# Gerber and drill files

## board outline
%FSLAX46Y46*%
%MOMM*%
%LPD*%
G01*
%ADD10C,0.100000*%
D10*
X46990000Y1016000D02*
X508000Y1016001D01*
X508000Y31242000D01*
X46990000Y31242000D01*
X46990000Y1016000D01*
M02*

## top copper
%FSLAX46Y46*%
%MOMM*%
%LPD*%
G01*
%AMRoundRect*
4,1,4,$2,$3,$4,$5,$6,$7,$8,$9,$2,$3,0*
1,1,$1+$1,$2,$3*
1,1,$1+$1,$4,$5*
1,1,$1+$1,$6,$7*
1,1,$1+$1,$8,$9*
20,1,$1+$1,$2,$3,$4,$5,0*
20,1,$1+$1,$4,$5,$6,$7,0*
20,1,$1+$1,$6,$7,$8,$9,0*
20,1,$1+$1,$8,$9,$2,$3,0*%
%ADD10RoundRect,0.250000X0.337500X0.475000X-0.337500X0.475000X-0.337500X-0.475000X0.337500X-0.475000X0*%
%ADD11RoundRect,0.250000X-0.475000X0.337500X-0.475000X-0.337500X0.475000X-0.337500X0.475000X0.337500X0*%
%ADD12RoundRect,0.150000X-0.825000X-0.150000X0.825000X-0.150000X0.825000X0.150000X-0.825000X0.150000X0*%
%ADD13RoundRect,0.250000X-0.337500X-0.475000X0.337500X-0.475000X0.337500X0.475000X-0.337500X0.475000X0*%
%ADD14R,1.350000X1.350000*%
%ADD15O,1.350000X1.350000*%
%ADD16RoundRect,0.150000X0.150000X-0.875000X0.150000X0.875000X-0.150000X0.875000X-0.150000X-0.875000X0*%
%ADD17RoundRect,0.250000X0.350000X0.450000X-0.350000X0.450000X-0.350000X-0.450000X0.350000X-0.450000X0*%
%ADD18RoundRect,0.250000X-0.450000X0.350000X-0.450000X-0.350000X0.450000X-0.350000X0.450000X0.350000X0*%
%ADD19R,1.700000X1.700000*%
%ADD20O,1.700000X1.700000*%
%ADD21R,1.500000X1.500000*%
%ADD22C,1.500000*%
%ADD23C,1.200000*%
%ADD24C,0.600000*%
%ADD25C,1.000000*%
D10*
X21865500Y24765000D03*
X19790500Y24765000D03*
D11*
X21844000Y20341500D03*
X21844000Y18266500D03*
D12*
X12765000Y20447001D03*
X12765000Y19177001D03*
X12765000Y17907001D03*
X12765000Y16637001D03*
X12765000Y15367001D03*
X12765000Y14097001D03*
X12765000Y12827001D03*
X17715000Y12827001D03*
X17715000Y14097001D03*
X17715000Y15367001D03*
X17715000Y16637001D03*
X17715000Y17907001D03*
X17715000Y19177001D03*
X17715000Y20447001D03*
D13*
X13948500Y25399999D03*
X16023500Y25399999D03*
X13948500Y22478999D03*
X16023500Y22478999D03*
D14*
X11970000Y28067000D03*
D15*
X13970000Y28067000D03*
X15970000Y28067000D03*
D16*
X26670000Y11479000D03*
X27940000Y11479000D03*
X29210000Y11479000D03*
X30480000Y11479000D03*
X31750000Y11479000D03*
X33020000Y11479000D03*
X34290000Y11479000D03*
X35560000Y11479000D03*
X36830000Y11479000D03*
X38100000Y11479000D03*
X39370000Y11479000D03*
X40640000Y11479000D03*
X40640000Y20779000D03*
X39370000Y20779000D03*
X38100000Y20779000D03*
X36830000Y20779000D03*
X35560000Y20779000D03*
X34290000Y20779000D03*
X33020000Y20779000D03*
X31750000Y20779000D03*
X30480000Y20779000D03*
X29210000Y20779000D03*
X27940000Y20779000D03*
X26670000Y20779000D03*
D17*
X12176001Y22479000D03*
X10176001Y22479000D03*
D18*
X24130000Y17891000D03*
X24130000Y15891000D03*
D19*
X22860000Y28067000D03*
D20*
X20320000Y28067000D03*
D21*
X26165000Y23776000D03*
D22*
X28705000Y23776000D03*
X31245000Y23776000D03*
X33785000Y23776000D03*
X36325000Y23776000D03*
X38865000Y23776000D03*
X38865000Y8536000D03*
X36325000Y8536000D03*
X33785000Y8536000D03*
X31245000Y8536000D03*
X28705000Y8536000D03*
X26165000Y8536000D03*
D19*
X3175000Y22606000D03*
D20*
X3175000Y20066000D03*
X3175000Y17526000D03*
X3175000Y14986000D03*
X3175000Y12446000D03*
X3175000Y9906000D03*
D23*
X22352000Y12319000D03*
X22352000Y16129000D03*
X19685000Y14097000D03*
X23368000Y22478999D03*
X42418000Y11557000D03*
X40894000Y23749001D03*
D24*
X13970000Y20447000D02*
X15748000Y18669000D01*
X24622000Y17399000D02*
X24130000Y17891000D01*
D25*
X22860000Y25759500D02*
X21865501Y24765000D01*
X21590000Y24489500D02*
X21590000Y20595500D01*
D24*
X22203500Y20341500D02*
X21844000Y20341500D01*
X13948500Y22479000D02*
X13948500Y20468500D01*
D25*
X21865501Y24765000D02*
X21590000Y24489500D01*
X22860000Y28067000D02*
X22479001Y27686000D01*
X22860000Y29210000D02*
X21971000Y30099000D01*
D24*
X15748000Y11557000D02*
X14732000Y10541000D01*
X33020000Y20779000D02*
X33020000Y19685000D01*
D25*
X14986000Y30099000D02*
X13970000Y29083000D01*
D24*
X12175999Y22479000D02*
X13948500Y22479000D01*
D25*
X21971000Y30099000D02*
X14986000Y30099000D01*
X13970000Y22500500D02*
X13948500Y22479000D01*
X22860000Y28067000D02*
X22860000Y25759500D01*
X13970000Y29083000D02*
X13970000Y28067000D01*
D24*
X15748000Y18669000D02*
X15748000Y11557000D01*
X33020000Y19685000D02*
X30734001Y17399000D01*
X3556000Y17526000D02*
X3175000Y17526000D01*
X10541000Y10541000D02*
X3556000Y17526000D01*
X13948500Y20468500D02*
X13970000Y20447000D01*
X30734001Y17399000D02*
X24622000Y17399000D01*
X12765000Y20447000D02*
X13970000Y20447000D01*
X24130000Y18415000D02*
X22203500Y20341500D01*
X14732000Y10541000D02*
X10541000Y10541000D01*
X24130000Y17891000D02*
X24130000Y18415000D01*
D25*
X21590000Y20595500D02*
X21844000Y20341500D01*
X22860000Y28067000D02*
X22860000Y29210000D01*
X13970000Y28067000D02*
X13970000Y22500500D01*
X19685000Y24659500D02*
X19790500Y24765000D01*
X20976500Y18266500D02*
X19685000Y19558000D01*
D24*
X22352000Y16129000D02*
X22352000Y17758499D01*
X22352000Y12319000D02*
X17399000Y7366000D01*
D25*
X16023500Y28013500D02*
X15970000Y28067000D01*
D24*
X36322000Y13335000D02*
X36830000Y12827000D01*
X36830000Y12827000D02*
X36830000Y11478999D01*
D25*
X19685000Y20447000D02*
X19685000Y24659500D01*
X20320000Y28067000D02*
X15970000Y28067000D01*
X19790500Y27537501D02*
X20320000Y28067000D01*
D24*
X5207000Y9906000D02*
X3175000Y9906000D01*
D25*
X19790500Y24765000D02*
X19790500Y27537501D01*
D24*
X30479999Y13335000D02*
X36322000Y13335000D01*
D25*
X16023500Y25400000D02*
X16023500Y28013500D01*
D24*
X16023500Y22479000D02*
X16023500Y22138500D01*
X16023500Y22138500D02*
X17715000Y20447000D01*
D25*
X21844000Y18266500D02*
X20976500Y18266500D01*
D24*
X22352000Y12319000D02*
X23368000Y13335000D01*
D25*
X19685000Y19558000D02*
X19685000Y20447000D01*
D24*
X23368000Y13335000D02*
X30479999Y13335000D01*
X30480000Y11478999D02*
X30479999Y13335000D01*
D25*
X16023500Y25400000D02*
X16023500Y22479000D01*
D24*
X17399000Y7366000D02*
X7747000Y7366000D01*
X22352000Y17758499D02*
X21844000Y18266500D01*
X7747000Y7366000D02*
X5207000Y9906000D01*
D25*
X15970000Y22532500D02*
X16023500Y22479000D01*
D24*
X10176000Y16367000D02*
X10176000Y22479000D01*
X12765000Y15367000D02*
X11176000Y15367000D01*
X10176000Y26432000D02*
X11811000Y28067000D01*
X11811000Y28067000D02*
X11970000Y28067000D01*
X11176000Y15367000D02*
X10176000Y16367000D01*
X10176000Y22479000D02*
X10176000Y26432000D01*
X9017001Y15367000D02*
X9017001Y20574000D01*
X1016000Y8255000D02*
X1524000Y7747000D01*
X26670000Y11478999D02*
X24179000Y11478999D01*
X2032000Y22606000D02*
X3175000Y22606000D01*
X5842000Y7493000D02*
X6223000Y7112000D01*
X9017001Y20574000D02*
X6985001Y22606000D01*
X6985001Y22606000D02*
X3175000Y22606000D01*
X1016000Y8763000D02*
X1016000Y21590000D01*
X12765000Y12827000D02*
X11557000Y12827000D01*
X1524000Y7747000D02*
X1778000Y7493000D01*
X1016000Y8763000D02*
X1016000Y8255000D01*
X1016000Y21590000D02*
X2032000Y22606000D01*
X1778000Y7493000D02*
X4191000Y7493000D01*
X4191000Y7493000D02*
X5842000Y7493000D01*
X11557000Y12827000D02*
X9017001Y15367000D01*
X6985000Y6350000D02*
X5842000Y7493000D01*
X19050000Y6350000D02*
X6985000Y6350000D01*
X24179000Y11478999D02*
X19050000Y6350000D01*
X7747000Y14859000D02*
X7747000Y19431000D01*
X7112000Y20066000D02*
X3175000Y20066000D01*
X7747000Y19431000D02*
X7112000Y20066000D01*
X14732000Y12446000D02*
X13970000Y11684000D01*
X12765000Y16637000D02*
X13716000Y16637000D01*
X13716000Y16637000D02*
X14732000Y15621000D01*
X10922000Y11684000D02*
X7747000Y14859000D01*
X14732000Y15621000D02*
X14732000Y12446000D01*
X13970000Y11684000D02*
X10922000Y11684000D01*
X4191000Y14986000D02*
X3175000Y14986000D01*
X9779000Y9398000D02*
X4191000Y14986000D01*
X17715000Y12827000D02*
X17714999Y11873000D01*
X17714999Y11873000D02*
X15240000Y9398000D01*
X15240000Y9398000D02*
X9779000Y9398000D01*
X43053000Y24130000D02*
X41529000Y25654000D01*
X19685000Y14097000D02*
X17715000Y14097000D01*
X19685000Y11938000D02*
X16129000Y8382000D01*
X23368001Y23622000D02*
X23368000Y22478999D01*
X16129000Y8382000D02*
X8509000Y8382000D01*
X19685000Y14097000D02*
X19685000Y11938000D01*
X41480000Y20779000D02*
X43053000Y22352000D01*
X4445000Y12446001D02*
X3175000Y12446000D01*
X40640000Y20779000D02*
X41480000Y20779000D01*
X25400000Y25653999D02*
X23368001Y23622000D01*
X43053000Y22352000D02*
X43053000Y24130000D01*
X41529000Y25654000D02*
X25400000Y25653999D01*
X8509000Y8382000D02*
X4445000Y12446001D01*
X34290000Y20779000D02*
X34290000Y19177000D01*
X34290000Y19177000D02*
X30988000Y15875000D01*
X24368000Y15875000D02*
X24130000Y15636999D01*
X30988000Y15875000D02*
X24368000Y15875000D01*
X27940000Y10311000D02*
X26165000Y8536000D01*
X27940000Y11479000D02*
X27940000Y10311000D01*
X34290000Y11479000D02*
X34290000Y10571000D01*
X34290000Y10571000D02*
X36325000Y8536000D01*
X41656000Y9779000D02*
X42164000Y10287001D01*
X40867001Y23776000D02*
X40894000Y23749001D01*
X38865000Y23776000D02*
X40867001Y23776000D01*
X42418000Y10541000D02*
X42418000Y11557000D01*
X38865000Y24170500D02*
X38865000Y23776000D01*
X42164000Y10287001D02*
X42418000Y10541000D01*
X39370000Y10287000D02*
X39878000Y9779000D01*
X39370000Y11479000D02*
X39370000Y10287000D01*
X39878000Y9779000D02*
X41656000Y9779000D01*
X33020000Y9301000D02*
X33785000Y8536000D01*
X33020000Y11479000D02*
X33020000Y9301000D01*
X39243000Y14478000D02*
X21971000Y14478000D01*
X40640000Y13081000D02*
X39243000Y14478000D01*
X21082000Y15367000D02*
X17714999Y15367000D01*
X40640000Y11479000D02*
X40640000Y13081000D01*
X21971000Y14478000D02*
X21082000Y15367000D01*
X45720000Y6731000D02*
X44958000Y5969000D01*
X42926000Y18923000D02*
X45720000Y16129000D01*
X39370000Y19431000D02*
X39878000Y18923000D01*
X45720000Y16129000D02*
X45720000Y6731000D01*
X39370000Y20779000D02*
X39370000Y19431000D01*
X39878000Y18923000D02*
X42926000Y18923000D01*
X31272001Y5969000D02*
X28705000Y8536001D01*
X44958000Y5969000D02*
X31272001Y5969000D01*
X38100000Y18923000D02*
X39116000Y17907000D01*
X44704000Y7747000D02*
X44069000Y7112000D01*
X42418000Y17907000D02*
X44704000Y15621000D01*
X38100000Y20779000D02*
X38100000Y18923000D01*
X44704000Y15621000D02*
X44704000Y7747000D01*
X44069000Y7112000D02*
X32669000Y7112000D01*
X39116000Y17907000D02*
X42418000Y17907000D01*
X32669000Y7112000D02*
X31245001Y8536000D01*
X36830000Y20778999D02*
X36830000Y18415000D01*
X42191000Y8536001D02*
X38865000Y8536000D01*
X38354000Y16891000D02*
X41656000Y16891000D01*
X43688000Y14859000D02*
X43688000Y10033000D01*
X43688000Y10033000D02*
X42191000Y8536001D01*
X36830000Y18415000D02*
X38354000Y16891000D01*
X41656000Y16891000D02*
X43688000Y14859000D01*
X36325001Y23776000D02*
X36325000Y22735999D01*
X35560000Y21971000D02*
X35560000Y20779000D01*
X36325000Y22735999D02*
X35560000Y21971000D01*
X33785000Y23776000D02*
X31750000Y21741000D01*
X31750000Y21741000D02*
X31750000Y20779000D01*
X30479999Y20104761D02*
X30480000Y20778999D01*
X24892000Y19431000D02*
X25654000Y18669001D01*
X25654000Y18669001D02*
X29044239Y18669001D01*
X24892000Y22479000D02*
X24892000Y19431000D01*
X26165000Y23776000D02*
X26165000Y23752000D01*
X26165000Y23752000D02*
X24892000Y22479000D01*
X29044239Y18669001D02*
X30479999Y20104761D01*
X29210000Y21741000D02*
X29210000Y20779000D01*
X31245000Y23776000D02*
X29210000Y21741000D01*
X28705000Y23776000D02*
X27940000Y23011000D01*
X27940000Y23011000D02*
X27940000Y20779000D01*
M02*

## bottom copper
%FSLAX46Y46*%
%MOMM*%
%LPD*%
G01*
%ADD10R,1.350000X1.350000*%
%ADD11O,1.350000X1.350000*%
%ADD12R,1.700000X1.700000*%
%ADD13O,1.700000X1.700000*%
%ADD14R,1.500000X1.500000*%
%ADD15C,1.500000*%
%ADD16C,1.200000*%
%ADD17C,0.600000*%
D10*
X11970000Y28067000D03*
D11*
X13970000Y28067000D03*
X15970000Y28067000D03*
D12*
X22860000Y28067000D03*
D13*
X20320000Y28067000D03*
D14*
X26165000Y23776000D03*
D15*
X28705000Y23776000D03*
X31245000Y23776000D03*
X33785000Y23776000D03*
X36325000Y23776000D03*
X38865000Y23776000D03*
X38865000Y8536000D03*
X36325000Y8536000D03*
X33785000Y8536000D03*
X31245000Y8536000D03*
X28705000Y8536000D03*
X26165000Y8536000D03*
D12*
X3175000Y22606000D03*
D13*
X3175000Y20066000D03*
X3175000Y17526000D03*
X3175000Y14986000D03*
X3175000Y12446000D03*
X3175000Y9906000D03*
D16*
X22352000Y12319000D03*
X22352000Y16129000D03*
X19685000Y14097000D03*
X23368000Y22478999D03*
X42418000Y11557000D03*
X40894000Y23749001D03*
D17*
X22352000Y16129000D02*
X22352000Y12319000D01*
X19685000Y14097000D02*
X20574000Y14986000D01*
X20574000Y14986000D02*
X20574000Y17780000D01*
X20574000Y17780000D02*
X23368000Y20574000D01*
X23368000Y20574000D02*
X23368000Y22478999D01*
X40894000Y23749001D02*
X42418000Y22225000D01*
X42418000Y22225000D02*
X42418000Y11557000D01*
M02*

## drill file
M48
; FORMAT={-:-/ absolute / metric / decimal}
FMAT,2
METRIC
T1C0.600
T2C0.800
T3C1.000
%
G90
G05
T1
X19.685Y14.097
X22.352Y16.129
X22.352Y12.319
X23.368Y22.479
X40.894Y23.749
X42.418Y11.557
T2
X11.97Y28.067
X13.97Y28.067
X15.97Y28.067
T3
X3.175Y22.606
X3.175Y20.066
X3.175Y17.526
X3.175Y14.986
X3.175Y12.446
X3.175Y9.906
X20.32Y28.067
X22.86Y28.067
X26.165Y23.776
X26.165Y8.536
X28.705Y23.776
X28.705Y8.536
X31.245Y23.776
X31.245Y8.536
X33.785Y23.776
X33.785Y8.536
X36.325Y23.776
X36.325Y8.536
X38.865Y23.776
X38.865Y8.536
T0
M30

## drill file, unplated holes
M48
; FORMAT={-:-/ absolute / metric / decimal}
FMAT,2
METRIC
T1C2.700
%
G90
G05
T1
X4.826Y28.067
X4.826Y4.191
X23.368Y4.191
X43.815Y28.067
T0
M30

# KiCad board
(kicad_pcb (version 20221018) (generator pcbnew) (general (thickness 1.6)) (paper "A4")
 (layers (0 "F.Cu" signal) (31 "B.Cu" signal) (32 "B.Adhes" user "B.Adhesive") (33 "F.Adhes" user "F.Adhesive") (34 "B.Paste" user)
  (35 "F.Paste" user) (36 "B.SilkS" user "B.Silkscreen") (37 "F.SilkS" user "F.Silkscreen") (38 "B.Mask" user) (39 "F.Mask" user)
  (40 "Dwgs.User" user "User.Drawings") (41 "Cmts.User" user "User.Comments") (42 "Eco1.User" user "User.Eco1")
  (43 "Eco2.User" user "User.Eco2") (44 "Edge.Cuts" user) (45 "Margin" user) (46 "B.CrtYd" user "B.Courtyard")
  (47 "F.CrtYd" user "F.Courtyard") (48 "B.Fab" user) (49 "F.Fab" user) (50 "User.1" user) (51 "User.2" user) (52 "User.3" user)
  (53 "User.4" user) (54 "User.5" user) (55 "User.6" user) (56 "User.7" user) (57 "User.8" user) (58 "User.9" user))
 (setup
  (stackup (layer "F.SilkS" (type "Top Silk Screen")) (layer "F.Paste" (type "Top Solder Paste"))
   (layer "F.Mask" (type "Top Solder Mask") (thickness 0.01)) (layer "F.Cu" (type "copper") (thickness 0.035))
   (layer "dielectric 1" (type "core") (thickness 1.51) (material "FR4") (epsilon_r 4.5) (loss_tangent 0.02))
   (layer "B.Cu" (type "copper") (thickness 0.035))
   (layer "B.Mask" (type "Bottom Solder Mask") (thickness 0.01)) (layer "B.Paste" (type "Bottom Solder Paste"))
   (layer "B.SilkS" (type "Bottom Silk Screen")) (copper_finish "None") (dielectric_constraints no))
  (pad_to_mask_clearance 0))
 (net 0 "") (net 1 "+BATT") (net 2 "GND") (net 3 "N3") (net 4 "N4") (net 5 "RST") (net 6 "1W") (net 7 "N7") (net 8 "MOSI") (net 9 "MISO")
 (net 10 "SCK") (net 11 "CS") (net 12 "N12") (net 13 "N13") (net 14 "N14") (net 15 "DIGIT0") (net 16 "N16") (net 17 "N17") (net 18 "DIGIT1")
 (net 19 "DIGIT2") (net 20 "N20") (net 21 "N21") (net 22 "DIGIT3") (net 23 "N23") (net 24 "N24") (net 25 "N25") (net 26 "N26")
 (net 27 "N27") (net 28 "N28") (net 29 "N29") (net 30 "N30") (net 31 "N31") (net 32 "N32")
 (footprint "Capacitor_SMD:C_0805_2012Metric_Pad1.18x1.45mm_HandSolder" (layer "F.Cu") (at 20.828 -24.765 180)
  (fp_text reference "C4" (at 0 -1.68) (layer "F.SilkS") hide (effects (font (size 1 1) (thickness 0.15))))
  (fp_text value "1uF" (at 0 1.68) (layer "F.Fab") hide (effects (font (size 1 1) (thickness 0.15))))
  (pad "1" smd roundrect (at -1.0375 0 180) (size 1.175 1.45) (layers "F.Cu" "F.Paste" "F.Mask") (roundrect_rratio 0.2127659574)
   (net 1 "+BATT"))
  (pad "2" smd roundrect (at 1.0375 0 180) (size 1.175 1.45) (layers "F.Cu" "F.Paste" "F.Mask") (roundrect_rratio 0.2127659574)
   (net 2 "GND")))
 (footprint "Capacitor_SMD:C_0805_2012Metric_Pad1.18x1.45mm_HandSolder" (layer "F.Cu") (at 21.844 -19.304 -90)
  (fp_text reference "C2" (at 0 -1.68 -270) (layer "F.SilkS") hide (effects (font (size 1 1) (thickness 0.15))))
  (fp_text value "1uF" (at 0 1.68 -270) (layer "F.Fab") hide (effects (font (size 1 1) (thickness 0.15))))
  (pad "1" smd roundrect (at -1.0375 0 270) (size 1.175 1.45) (layers "F.Cu" "F.Paste" "F.Mask") (roundrect_rratio 0.2127659574)
   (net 1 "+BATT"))
  (pad "2" smd roundrect (at 1.0375 0 270) (size 1.175 1.45) (layers "F.Cu" "F.Paste" "F.Mask") (roundrect_rratio 0.2127659574)
   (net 2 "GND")))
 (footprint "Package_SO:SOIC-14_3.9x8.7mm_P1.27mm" (layer "F.Cu") (at 15.24 -16.637001)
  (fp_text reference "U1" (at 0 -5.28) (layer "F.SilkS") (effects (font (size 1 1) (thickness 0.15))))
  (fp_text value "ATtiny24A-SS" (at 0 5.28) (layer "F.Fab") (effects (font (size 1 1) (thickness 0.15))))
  (pad "1" smd roundrect (at -2.475 -3.81) (size 1.95 0.6) (layers "F.Cu" "F.Paste" "F.Mask") (roundrect_rratio 0.25) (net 1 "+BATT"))
  (pad "2" smd roundrect (at -2.475 -2.54) (size 1.95 0.6) (layers "F.Cu" "F.Paste" "F.Mask") (roundrect_rratio 0.25) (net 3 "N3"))
  (pad "3" smd roundrect (at -2.475 -1.27) (size 1.95 0.6) (layers "F.Cu" "F.Paste" "F.Mask") (roundrect_rratio 0.25) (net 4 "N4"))
  (pad "4" smd roundrect (at -2.475 0) (size 1.95 0.6) (layers "F.Cu" "F.Paste" "F.Mask") (roundrect_rratio 0.25) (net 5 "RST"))
  (pad "5" smd roundrect (at -2.475 1.27) (size 1.95 0.6) (layers "F.Cu" "F.Paste" "F.Mask") (roundrect_rratio 0.25) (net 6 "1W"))
  (pad "6" smd roundrect (at -2.475 2.54) (size 1.95 0.6) (layers "F.Cu" "F.Paste" "F.Mask") (roundrect_rratio 0.25) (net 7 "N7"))
  (pad "7" smd roundrect (at -2.475 3.81) (size 1.95 0.6) (layers "F.Cu" "F.Paste" "F.Mask") (roundrect_rratio 0.25) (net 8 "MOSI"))
  (pad "8" smd roundrect (at 2.475 3.81) (size 1.95 0.6) (layers "F.Cu" "F.Paste" "F.Mask") (roundrect_rratio 0.25) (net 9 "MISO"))
  (pad "9" smd roundrect (at 2.475 2.54) (size 1.95 0.6) (layers "F.Cu" "F.Paste" "F.Mask") (roundrect_rratio 0.25) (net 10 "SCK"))
  (pad "10" smd roundrect (at 2.475 1.27) (size 1.95 0.6) (layers "F.Cu" "F.Paste" "F.Mask") (roundrect_rratio 0.25) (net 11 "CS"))
  (pad "11" smd roundrect (at 2.475 0) (size 1.95 0.6) (layers "F.Cu" "F.Paste" "F.Mask") (roundrect_rratio 0.25) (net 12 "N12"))
  (pad "12" smd roundrect (at 2.475 -1.27) (size 1.95 0.6) (layers "F.Cu" "F.Paste" "F.Mask") (roundrect_rratio 0.25) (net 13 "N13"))
  (pad "13" smd roundrect (at 2.475 -2.54) (size 1.95 0.6) (layers "F.Cu" "F.Paste" "F.Mask") (roundrect_rratio 0.25) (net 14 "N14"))
  (pad "14" smd roundrect (at 2.475 -3.81) (size 1.95 0.6) (layers "F.Cu" "F.Paste" "F.Mask") (roundrect_rratio 0.25) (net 2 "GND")))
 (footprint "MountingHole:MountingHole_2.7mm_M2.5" (layer "F.Cu") (at 43.815 -28.067 90)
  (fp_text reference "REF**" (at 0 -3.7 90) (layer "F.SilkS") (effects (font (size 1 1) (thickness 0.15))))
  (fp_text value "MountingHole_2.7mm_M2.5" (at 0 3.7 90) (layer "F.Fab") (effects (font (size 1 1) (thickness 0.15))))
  (pad "" np_thru_hole circle (at 0 0 90) (size 2.7 2.7) (drill 2.7) (layers "F&B.Cu" "*.Mask")))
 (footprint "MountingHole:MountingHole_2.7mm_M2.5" (layer "F.Cu") (at 23.368 -4.191001 90)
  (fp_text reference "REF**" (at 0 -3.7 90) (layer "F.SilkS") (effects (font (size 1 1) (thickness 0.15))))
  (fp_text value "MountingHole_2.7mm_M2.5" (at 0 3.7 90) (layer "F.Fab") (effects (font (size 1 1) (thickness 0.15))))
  (pad "" np_thru_hole circle (at 0 0 90) (size 2.7 2.7) (drill 2.7) (layers "F&B.Cu" "*.Mask")))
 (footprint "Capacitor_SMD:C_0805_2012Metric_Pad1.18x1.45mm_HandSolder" (layer "F.Cu") (at 14.986 -25.399999)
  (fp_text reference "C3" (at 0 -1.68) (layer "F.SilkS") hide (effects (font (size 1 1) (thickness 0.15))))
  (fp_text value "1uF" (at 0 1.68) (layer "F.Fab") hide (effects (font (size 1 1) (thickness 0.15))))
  (pad "1" smd roundrect (at -1.0375 0) (size 1.175 1.45) (layers "F.Cu" "F.Paste" "F.Mask") (roundrect_rratio 0.2127659574) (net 1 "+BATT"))
  (pad "2" smd roundrect (at 1.0375 0) (size 1.175 1.45) (layers "F.Cu" "F.Paste" "F.Mask") (roundrect_rratio 0.2127659574) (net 2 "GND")))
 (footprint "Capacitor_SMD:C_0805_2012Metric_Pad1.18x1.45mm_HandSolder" (layer "F.Cu") (at 14.986 -22.478999)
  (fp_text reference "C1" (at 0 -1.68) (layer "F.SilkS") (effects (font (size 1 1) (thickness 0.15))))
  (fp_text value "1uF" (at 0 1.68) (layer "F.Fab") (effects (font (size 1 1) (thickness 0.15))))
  (pad "1" smd roundrect (at -1.0375 0) (size 1.175 1.45) (layers "F.Cu" "F.Paste" "F.Mask") (roundrect_rratio 0.2127659574) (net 1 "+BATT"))
  (pad "2" smd roundrect (at 1.0375 0) (size 1.175 1.45) (layers "F.Cu" "F.Paste" "F.Mask") (roundrect_rratio 0.2127659574) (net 2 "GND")))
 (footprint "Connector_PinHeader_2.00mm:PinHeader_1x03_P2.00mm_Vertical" (layer "F.Cu") (at 11.97 -28.067 90)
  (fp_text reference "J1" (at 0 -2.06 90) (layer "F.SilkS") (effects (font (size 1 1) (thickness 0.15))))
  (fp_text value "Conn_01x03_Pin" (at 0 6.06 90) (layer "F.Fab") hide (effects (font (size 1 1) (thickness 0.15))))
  (pad "1" thru_hole rect (at 0 0 90) (size 1.35 1.35) (drill 0.8) (layers "*.Cu" "*.Mask") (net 6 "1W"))
  (pad "2" thru_hole oval (at 0 2 90) (size 1.35 1.35) (drill 0.8) (layers "*.Cu" "*.Mask") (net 1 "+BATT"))
  (pad "3" thru_hole oval (at 0 4 90) (size 1.35 1.35) (drill 0.8) (layers "*.Cu" "*.Mask") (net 2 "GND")))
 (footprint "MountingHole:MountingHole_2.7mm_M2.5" (layer "F.Cu") (at 4.826 -4.191001 90)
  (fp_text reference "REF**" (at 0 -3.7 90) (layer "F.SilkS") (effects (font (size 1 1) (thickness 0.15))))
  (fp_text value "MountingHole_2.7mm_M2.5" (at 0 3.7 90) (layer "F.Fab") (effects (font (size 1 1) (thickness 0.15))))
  (pad "" np_thru_hole circle (at 0 0 90) (size 2.7 2.7) (drill 2.7) (layers "*.Cu" "*.Mask")))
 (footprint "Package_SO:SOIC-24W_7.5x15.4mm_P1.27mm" (layer "F.Cu") (at 33.655 -16.129 90)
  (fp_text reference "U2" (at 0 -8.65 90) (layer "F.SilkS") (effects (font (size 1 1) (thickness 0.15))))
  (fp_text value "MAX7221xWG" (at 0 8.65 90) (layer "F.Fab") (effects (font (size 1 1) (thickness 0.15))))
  (pad "1" smd roundrect (at -4.65 -6.985 90) (size 2.05 0.6) (layers "F.Cu" "F.Paste" "F.Mask") (roundrect_rratio 0.25) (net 8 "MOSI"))
  (pad "2" smd roundrect (at -4.65 -5.715 90) (size 2.05 0.6) (layers "F.Cu" "F.Paste" "F.Mask") (roundrect_rratio 0.25) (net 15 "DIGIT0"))
  (pad "3" smd roundrect (at -4.65 -4.445 90) (size 2.05 0.6) (layers "F.Cu" "F.Paste" "F.Mask") (roundrect_rratio 0.25) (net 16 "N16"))
  (pad "4" smd roundrect (at -4.65 -3.175 90) (size 2.05 0.6) (layers "F.Cu" "F.Paste" "F.Mask") (roundrect_rratio 0.25) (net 2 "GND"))
  (pad "5" smd roundrect (at -4.65 -1.905 90) (size 2.05 0.6) (layers "F.Cu" "F.Paste" "F.Mask") (roundrect_rratio 0.25) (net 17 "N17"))
  (pad "6" smd roundrect (at -4.65 -0.635 90) (size 2.05 0.6) (layers "F.Cu" "F.Paste" "F.Mask") (roundrect_rratio 0.25) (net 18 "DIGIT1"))
  (pad "7" smd roundrect (at -4.65 0.635 90) (size 2.05 0.6) (layers "F.Cu" "F.Paste" "F.Mask") (roundrect_rratio 0.25) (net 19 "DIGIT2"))
  (pad "8" smd roundrect (at -4.65 1.905 90) (size 2.05 0.6) (layers "F.Cu" "F.Paste" "F.Mask") (roundrect_rratio 0.25) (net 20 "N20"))
  (pad "9" smd roundrect (at -4.65 3.175 90) (size 2.05 0.6) (layers "F.Cu" "F.Paste" "F.Mask") (roundrect_rratio 0.25) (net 2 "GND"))
  (pad "10" smd roundrect (at -4.65 4.445 90) (size 2.05 0.6) (layers "F.Cu" "F.Paste" "F.Mask") (roundrect_rratio 0.25) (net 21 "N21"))
  (pad "11" smd roundrect (at -4.65 5.715 90) (size 2.05 0.6) (layers "F.Cu" "F.Paste" "F.Mask") (roundrect_rratio 0.25) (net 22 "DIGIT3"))
  (pad "12" smd roundrect (at -4.65 6.985 90) (size 2.05 0.6) (layers "F.Cu" "F.Paste" "F.Mask") (roundrect_rratio 0.25) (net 11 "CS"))
  (pad "13" smd roundrect (at 4.65 6.985 90) (size 2.05 0.6) (layers "F.Cu" "F.Paste" "F.Mask") (roundrect_rratio 0.25) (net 10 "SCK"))
  (pad "14" smd roundrect (at 4.65 5.715 90) (size 2.05 0.6) (layers "F.Cu" "F.Paste" "F.Mask") (roundrect_rratio 0.25) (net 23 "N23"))
  (pad "15" smd roundrect (at 4.65 4.445 90) (size 2.05 0.6) (layers "F.Cu" "F.Paste" "F.Mask") (roundrect_rratio 0.25) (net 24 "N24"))
  (pad "16" smd roundrect (at 4.65 3.175 90) (size 2.05 0.6) (layers "F.Cu" "F.Paste" "F.Mask") (roundrect_rratio 0.25) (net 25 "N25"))
  (pad "17" smd roundrect (at 4.65 1.905 90) (size 2.05 0.6) (layers "F.Cu" "F.Paste" "F.Mask") (roundrect_rratio 0.25) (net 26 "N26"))
  (pad "18" smd roundrect (at 4.65 0.635 90) (size 2.05 0.6) (layers "F.Cu" "F.Paste" "F.Mask") (roundrect_rratio 0.25) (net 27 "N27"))
  (pad "19" smd roundrect (at 4.65 -0.635 90) (size 2.05 0.6) (layers "F.Cu" "F.Paste" "F.Mask") (roundrect_rratio 0.25) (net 1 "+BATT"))
  (pad "20" smd roundrect (at 4.65 -1.905 90) (size 2.05 0.6) (layers "F.Cu" "F.Paste" "F.Mask") (roundrect_rratio 0.25) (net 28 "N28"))
  (pad "21" smd roundrect (at 4.65 -3.175 90) (size 2.05 0.6) (layers "F.Cu" "F.Paste" "F.Mask") (roundrect_rratio 0.25) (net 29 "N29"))
  (pad "22" smd roundrect (at 4.65 -4.445 90) (size 2.05 0.6) (layers "F.Cu" "F.Paste" "F.Mask") (roundrect_rratio 0.25) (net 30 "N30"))
  (pad "23" smd roundrect (at 4.65 -5.715 90) (size 2.05 0.6) (layers "F.Cu" "F.Paste" "F.Mask") (roundrect_rratio 0.25) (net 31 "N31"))
  (pad "24" smd roundrect (at 4.65 -6.985 90) (size 2.05 0.6) (layers "F.Cu" "F.Paste" "F.Mask") (roundrect_rratio 0.25) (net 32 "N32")))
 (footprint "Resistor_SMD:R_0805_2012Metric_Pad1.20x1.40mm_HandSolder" (layer "F.Cu") (at 11.176001 -22.479 180)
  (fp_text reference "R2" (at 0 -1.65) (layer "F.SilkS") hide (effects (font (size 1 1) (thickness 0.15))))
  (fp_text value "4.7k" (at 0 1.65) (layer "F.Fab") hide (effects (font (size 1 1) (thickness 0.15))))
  (pad "1" smd roundrect (at -1 0 180) (size 1.2 1.4) (layers "F.Cu" "F.Paste" "F.Mask") (roundrect_rratio 0.2083333333) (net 1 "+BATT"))
  (pad "2" smd roundrect (at 1 0 180) (size 1.2 1.4) (layers "F.Cu" "F.Paste" "F.Mask") (roundrect_rratio 0.2083333333) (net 6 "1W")))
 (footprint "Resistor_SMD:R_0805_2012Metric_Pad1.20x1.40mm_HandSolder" (layer "F.Cu") (at 24.13 -16.891 -90)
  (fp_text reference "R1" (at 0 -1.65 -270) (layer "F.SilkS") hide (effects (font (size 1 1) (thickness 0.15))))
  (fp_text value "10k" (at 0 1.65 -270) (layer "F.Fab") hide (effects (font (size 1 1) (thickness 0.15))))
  (pad "1" smd roundrect (at -1 0 270) (size 1.2 1.4) (layers "F.Cu" "F.Paste" "F.Mask") (roundrect_rratio 0.2083333333) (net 1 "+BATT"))
  (pad "2" smd roundrect (at 1 0 270) (size 1.2 1.4) (layers "F.Cu" "F.Paste" "F.Mask") (roundrect_rratio 0.2083333333) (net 27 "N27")))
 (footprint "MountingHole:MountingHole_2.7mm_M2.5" (layer "F.Cu") (at 4.826 -28.067 90)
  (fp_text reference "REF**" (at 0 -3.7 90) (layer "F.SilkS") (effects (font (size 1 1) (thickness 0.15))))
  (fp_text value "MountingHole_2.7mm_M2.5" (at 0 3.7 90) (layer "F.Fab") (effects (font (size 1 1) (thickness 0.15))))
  (pad "" np_thru_hole circle (at 0 0 90) (size 2.7 2.7) (drill 2.7) (layers "*.Cu" "*.Mask")))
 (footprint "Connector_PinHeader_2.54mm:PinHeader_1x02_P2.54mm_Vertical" (layer "F.Cu") (at 22.86 -28.067 -90)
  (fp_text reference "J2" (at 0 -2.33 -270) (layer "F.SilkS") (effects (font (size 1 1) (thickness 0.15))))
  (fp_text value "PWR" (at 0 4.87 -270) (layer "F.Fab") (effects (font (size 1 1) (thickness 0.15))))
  (pad "1" thru_hole rect (at 0 0 270) (size 1.7 1.7) (drill 1) (layers "*.Cu" "*.Mask") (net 1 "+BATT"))
  (pad "2" thru_hole oval (at 0 2.54 270) (size 1.7 1.7) (drill 1) (layers "*.Cu" "*.Mask") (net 2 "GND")))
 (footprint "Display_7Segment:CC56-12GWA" (layer "B.Cu") (at 26.165 -23.776 -90)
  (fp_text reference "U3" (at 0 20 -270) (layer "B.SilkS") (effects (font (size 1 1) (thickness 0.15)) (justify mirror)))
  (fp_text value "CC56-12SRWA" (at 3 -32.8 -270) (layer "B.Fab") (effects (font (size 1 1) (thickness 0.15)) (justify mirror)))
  (pad "1" thru_hole rect (at 0 0 270) (size 1.5 1.5) (drill 1) (layers "*.Cu" "*.Mask") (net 29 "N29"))
  (pad "2" thru_hole circle (at 0 -2.54 270) (size 1.5 1.5) (drill 1) (layers "*.Cu" "*.Mask") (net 31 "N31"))
  (pad "3" thru_hole circle (at 0 -5.08 270) (size 1.5 1.5) (drill 1) (layers "*.Cu" "*.Mask") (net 30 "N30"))
  (pad "4" thru_hole circle (at 0 -7.62 270) (size 1.5 1.5) (drill 1) (layers "*.Cu" "*.Mask") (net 28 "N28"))
  (pad "5" thru_hole circle (at 0 -10.16 270) (size 1.5 1.5) (drill 1) (layers "*.Cu" "*.Mask") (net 26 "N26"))
  (pad "6" thru_hole circle (at 0 -12.7 270) (size 1.5 1.5) (drill 1) (layers "*.Cu" "*.Mask") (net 22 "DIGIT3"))
  (pad "7" thru_hole circle (at 15.24 -12.7 270) (size 1.5 1.5) (drill 1) (layers "*.Cu" "*.Mask") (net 25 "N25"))
  (pad "8" thru_hole circle (at 15.24 -10.16 270) (size 1.5 1.5) (drill 1) (layers "*.Cu" "*.Mask") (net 19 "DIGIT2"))
  (pad "9" thru_hole circle (at 15.24 -7.62 270) (size 1.5 1.5) (drill 1) (layers "*.Cu" "*.Mask") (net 18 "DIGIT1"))
  (pad "10" thru_hole circle (at 15.24 -5.08 270) (size 1.5 1.5) (drill 1) (layers "*.Cu" "*.Mask") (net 24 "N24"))
  (pad "11" thru_hole circle (at 15.24 -2.54 270) (size 1.5 1.5) (drill 1) (layers "*.Cu" "*.Mask") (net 23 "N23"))
  (pad "12" thru_hole circle (at 15.24 0 270) (size 1.5 1.5) (drill 1) (layers "*.Cu" "*.Mask") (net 15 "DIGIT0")))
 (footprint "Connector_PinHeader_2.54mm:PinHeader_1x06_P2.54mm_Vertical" (layer "B.Cu") (at 3.175 -22.606 180)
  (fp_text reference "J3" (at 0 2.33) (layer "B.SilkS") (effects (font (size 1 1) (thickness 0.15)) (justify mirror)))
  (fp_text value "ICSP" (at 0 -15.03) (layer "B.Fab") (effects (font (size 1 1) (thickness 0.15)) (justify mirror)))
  (pad "1" thru_hole rect (at 0 0 180) (size 1.7 1.7) (drill 1) (layers "*.Cu" "*.Mask") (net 8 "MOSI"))
  (pad "2" thru_hole oval (at 0 -2.54 180) (size 1.7 1.7) (drill 1) (layers "*.Cu" "*.Mask") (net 5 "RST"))
  (pad "3" thru_hole oval (at 0 -5.08 180) (size 1.7 1.7) (drill 1) (layers "*.Cu" "*.Mask") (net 1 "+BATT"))
  (pad "4" thru_hole oval (at 0 -7.62 180) (size 1.7 1.7) (drill 1) (layers "*.Cu" "*.Mask") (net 9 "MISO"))
  (pad "5" thru_hole oval (at 0 -10.16 180) (size 1.7 1.7) (drill 1) (layers "*.Cu" "*.Mask") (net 10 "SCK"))
  (pad "6" thru_hole oval (at 0 -12.7 180) (size 1.7 1.7) (drill 1) (layers "*.Cu" "*.Mask") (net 2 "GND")))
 (gr_poly
  (pts (xy 0.508 -1.016001) (xy 0.508 -31.242) (xy 46.99 -31.242) (xy 46.99 -1.016)) (stroke (width 0.1) (type default)) (fill none)
  (layer "Edge.Cuts"))
 (segment (start 13.97 -20.447) (end 15.748 -18.669) (width 0.6) (layer "F.Cu") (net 1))
 (segment (start 24.622 -17.399) (end 24.13 -17.891) (width 0.6) (layer "F.Cu") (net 1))
 (segment (start 22.86 -25.7595) (end 21.865501 -24.765) (width 1) (layer "F.Cu") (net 1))
 (segment (start 21.59 -24.4895) (end 21.59 -20.5955) (width 1) (layer "F.Cu") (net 1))
 (segment (start 22.2035 -20.3415) (end 21.844 -20.3415) (width 0.6) (layer "F.Cu") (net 1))
 (segment (start 13.9485 -22.479) (end 13.9485 -20.4685) (width 0.6) (layer "F.Cu") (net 1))
 (segment (start 21.865501 -24.765) (end 21.59 -24.4895) (width 1) (layer "F.Cu") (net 1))
 (segment (start 22.86 -28.067) (end 22.479001 -27.686) (width 1) (layer "F.Cu") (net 1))
 (segment (start 22.86 -29.21) (end 21.971 -30.099) (width 1) (layer "F.Cu") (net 1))
 (segment (start 15.748 -11.557) (end 14.732 -10.541) (width 0.6) (layer "F.Cu") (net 1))
 (segment (start 33.02 -20.779) (end 33.02 -19.685) (width 0.6) (layer "F.Cu") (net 1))
 (segment (start 14.986 -30.099) (end 13.97 -29.083) (width 1) (layer "F.Cu") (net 1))
 (segment (start 12.175999 -22.479) (end 13.9485 -22.479) (width 0.6) (layer "F.Cu") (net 1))
 (segment (start 21.971 -30.099) (end 14.986 -30.099) (width 1) (layer "F.Cu") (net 1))
 (segment (start 13.97 -22.5005) (end 13.9485 -22.479) (width 1) (layer "F.Cu") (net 1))
 (segment (start 22.86 -28.067) (end 22.86 -25.7595) (width 1) (layer "F.Cu") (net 1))
 (segment (start 13.97 -29.083) (end 13.97 -28.067) (width 1) (layer "F.Cu") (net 1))
 (segment (start 15.748 -18.669) (end 15.748 -11.557) (width 0.6) (layer "F.Cu") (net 1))
 (segment (start 33.02 -19.685) (end 30.734001 -17.399) (width 0.6) (layer "F.Cu") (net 1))
 (segment (start 3.556 -17.526) (end 3.175 -17.526) (width 0.6) (layer "F.Cu") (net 1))
 (segment (start 10.541 -10.541) (end 3.556 -17.526) (width 0.6) (layer "F.Cu") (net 1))
 (segment (start 13.9485 -20.4685) (end 13.97 -20.447) (width 0.6) (layer "F.Cu") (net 1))
 (segment (start 30.734001 -17.399) (end 24.622 -17.399) (width 0.6) (layer "F.Cu") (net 1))
 (segment (start 12.765 -20.447) (end 13.97 -20.447) (width 0.6) (layer "F.Cu") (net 1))
 (segment (start 24.13 -18.415) (end 22.2035 -20.3415) (width 0.6) (layer "F.Cu") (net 1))
 (segment (start 14.732 -10.541) (end 10.541 -10.541) (width 0.6) (layer "F.Cu") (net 1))
 (segment (start 24.13 -17.891) (end 24.13 -18.415) (width 0.6) (layer "F.Cu") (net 1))
 (segment (start 21.59 -20.5955) (end 21.844 -20.3415) (width 1) (layer "F.Cu") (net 1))
 (segment (start 22.86 -28.067) (end 22.86 -29.21) (width 1) (layer "F.Cu") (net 1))
 (segment (start 13.97 -28.067) (end 13.97 -22.5005) (width 1) (layer "F.Cu") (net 1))
 (segment (start 19.685 -24.6595) (end 19.7905 -24.765) (width 1) (layer "F.Cu") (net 2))
 (segment (start 20.9765 -18.2665) (end 19.685 -19.558) (width 1) (layer "F.Cu") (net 2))
 (segment (start 22.352 -16.129) (end 22.352 -17.758499) (width 0.6) (layer "F.Cu") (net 2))
 (segment (start 22.352 -12.319) (end 17.399 -7.366) (width 0.6) (layer "F.Cu") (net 2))
 (segment (start 16.0235 -28.0135) (end 15.97 -28.067) (width 1) (layer "F.Cu") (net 2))
 (segment (start 36.322 -13.335) (end 36.83 -12.827) (width 0.6) (layer "F.Cu") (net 2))
 (segment (start 36.83 -12.827) (end 36.83 -11.478999) (width 0.6) (layer "F.Cu") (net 2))
 (segment (start 19.685 -20.447) (end 19.685 -24.6595) (width 1) (layer "F.Cu") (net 2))
 (segment (start 20.32 -28.067) (end 15.97 -28.067) (width 1) (layer "F.Cu") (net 2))
 (segment (start 19.7905 -27.537501) (end 20.32 -28.067) (width 1) (layer "F.Cu") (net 2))
 (segment (start 5.207 -9.906) (end 3.175 -9.906) (width 0.6) (layer "F.Cu") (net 2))
 (segment (start 19.7905 -24.765) (end 19.7905 -27.537501) (width 1) (layer "F.Cu") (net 2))
 (segment (start 30.479999 -13.335) (end 36.322 -13.335) (width 0.6) (layer "F.Cu") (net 2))
 (segment (start 16.0235 -25.4) (end 16.0235 -28.0135) (width 1) (layer "F.Cu") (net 2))
 (segment (start 16.0235 -22.479) (end 16.0235 -22.1385) (width 0.6) (layer "F.Cu") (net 2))
 (segment (start 16.0235 -22.1385) (end 17.715 -20.447) (width 0.6) (layer "F.Cu") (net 2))
 (segment (start 21.844 -18.2665) (end 20.9765 -18.2665) (width 1) (layer "F.Cu") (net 2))
 (segment (start 22.352 -12.319) (end 23.368 -13.335) (width 0.6) (layer "F.Cu") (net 2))
 (segment (start 19.685 -19.558) (end 19.685 -20.447) (width 1) (layer "F.Cu") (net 2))
 (segment (start 23.368 -13.335) (end 30.479999 -13.335) (width 0.6) (layer "F.Cu") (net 2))
 (segment (start 30.48 -11.478999) (end 30.479999 -13.335) (width 0.6) (layer "F.Cu") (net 2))
 (segment (start 16.0235 -25.4) (end 16.0235 -22.479) (width 1) (layer "F.Cu") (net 2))
 (segment (start 17.399 -7.366) (end 7.747 -7.366) (width 0.6) (layer "F.Cu") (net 2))
 (segment (start 22.352 -17.758499) (end 21.844 -18.2665) (width 0.6) (layer "F.Cu") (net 2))
 (segment (start 7.747 -7.366) (end 5.207 -9.906) (width 0.6) (layer "F.Cu") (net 2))
 (segment (start 15.97 -22.5325) (end 16.0235 -22.479) (width 1) (layer "F.Cu") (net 2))
 (via (at 22.352 -12.319) (size 1.2) (drill 0.6) (layers "F.Cu" "B.Cu") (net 2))
 (via (at 22.352 -16.129) (size 1.2) (drill 0.6) (layers "F.Cu" "B.Cu") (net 2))
 (segment (start 22.352 -16.129) (end 22.352 -12.319) (width 0.6) (layer "B.Cu") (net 2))
 (segment (start 10.176 -16.367) (end 10.176 -22.479) (width 0.6) (layer "F.Cu") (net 6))
 (segment (start 12.765 -15.367) (end 11.176 -15.367) (width 0.6) (layer "F.Cu") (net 6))
 (segment (start 10.176 -26.432) (end 11.811 -28.067) (width 0.6) (layer "F.Cu") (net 6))
 (segment (start 11.811 -28.067) (end 11.97 -28.067) (width 0.6) (layer "F.Cu") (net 6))
 (segment (start 11.176 -15.367) (end 10.176 -16.367) (width 0.6) (layer "F.Cu") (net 6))
 (segment (start 10.176 -22.479) (end 10.176 -26.432) (width 0.6) (layer "F.Cu") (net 6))
 (segment (start 9.017001 -15.367) (end 9.017001 -20.574) (width 0.6) (layer "F.Cu") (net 8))
 (segment (start 1.016 -8.255) (end 1.524 -7.747) (width 0.6) (layer "F.Cu") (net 8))
 (segment (start 26.67 -11.478999) (end 24.179 -11.478999) (width 0.6) (layer "F.Cu") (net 8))
 (segment (start 2.032 -22.606) (end 3.175 -22.606) (width 0.6) (layer "F.Cu") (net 8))
 (segment (start 5.842 -7.493) (end 6.223 -7.112) (width 0.6) (layer "F.Cu") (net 8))
 (segment (start 9.017001 -20.574) (end 6.985001 -22.606) (width 0.6) (layer "F.Cu") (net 8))
 (segment (start 6.985001 -22.606) (end 3.175 -22.606) (width 0.6) (layer "F.Cu") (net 8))
 (segment (start 1.016 -8.763) (end 1.016 -21.59) (width 0.6) (layer "F.Cu") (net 8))
 (segment (start 12.765 -12.827) (end 11.557 -12.827) (width 0.6) (layer "F.Cu") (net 8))
 (segment (start 1.524 -7.747) (end 1.778 -7.493) (width 0.6) (layer "F.Cu") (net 8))
 (segment (start 1.016 -8.763) (end 1.016 -8.255) (width 0.6) (layer "F.Cu") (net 8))
 (segment (start 1.016 -21.59) (end 2.032 -22.606) (width 0.6) (layer "F.Cu") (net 8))
 (segment (start 1.778 -7.493) (end 4.191 -7.493) (width 0.6) (layer "F.Cu") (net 8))
 (segment (start 4.191 -7.493) (end 5.842 -7.493) (width 0.6) (layer "F.Cu") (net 8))
 (segment (start 11.557 -12.827) (end 9.017001 -15.367) (width 0.6) (layer "F.Cu") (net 8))
 (segment (start 6.985 -6.35) (end 5.842 -7.493) (width 0.6) (layer "F.Cu") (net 8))
 (segment (start 19.05 -6.35) (end 6.985 -6.35) (width 0.6) (layer "F.Cu") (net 8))
 (segment (start 24.179 -11.478999) (end 19.05 -6.35) (width 0.6) (layer "F.Cu") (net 8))
 (segment (start 7.747 -14.859) (end 7.747 -19.431) (width 0.6) (layer "F.Cu") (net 5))
 (segment (start 7.112 -20.066) (end 3.175 -20.066) (width 0.6) (layer "F.Cu") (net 5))
 (segment (start 7.747 -19.431) (end 7.112 -20.066) (width 0.6) (layer "F.Cu") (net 5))
 (segment (start 14.732 -12.446) (end 13.97 -11.684) (width 0.6) (layer "F.Cu") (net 5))
 (segment (start 12.765 -16.637) (end 13.716 -16.637) (width 0.6) (layer "F.Cu") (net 5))
 (segment (start 13.716 -16.637) (end 14.732 -15.621) (width 0.6) (layer "F.Cu") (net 5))
 (segment (start 10.922 -11.684) (end 7.747 -14.859) (width 0.6) (layer "F.Cu") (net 5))
 (segment (start 14.732 -15.621) (end 14.732 -12.446) (width 0.6) (layer "F.Cu") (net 5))
 (segment (start 13.97 -11.684) (end 10.922 -11.684) (width 0.6) (layer "F.Cu") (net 5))
 (segment (start 4.191 -14.986) (end 3.175 -14.986) (width 0.6) (layer "F.Cu") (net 9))
 (segment (start 9.779 -9.398) (end 4.191 -14.986) (width 0.6) (layer "F.Cu") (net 9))
 (segment (start 17.715 -12.827) (end 17.714999 -11.873) (width 0.6) (layer "F.Cu") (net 9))
 (segment (start 17.714999 -11.873) (end 15.24 -9.398) (width 0.6) (layer "F.Cu") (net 9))
 (segment (start 15.24 -9.398) (end 9.779 -9.398) (width 0.6) (layer "F.Cu") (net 9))
 (segment (start 43.053 -24.13) (end 41.529 -25.654) (width 0.6) (layer "F.Cu") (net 10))
 (segment (start 19.685 -14.097) (end 17.715 -14.097) (width 0.6) (layer "F.Cu") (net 10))
 (segment (start 19.685 -11.938) (end 16.129 -8.382) (width 0.6) (layer "F.Cu") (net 10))
 (segment (start 23.368001 -23.622) (end 23.368 -22.478999) (width 0.6) (layer "F.Cu") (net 10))
 (segment (start 16.129 -8.382) (end 8.509 -8.382) (width 0.6) (layer "F.Cu") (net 10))
 (segment (start 19.685 -14.097) (end 19.685 -11.938) (width 0.6) (layer "F.Cu") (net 10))
 (segment (start 41.48 -20.779) (end 43.053 -22.352) (width 0.6) (layer "F.Cu") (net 10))
 (segment (start 4.445 -12.446001) (end 3.175 -12.446) (width 0.6) (layer "F.Cu") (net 10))
 (segment (start 40.64 -20.779) (end 41.48 -20.779) (width 0.6) (layer "F.Cu") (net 10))
 (segment (start 25.4 -25.653999) (end 23.368001 -23.622) (width 0.6) (layer "F.Cu") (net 10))
 (segment (start 43.053 -22.352) (end 43.053 -24.13) (width 0.6) (layer "F.Cu") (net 10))
 (segment (start 41.529 -25.654) (end 25.4 -25.653999) (width 0.6) (layer "F.Cu") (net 10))
 (segment (start 8.509 -8.382) (end 4.445 -12.446001) (width 0.6) (layer "F.Cu") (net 10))
 (via (at 19.685 -14.097) (size 1.2) (drill 0.6) (layers "F.Cu" "B.Cu") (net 10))
 (via (at 23.368 -22.478999) (size 1.2) (drill 0.6) (layers "F.Cu" "B.Cu") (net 10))
 (segment (start 19.685 -14.097) (end 20.574 -14.986) (width 0.6) (layer "B.Cu") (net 10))
 (segment (start 20.574 -14.986) (end 20.574 -17.78) (width 0.6) (layer "B.Cu") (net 10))
 (segment (start 20.574 -17.78) (end 23.368 -20.574) (width 0.6) (layer "B.Cu") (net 10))
 (segment (start 23.368 -20.574) (end 23.368 -22.478999) (width 0.6) (layer "B.Cu") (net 10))
 (segment (start 34.29 -20.779) (end 34.29 -19.177) (width 0.6) (layer "F.Cu") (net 27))
 (segment (start 34.29 -19.177) (end 30.988 -15.875) (width 0.6) (layer "F.Cu") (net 27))
 (segment (start 24.368 -15.875) (end 24.13 -15.636999) (width 0.6) (layer "F.Cu") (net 27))
 (segment (start 30.988 -15.875) (end 24.368 -15.875) (width 0.6) (layer "F.Cu") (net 27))
 (segment (start 27.94 -10.311) (end 26.165 -8.536) (width 0.6) (layer "F.Cu") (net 15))
 (segment (start 27.94 -11.479) (end 27.94 -10.311) (width 0.6) (layer "F.Cu") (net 15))
 (segment (start 34.29 -11.479) (end 34.29 -10.571) (width 0.6) (layer "F.Cu") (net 19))
 (segment (start 34.29 -10.571) (end 36.325 -8.536) (width 0.6) (layer "F.Cu") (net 19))
 (segment (start 41.656 -9.779) (end 42.164 -10.287001) (width 0.6) (layer "F.Cu") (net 22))
 (segment (start 40.867001 -23.776) (end 40.894 -23.749001) (width 0.6) (layer "F.Cu") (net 22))
 (segment (start 38.865 -23.776) (end 40.867001 -23.776) (width 0.6) (layer "F.Cu") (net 22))
 (segment (start 42.418 -10.541) (end 42.418 -11.557) (width 0.6) (layer "F.Cu") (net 22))
 (segment (start 38.865 -24.1705) (end 38.865 -23.776) (width 0.6) (layer "F.Cu") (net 22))
 (segment (start 42.164 -10.287001) (end 42.418 -10.541) (width 0.6) (layer "F.Cu") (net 22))
 (segment (start 39.37 -10.287) (end 39.878 -9.779) (width 0.6) (layer "F.Cu") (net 22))
 (segment (start 39.37 -11.479) (end 39.37 -10.287) (width 0.6) (layer "F.Cu") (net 22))
 (segment (start 39.878 -9.779) (end 41.656 -9.779) (width 0.6) (layer "F.Cu") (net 22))
 (via (at 42.418 -11.557) (size 1.2) (drill 0.6) (layers "F.Cu" "B.Cu") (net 22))
 (via (at 40.894 -23.749001) (size 1.2) (drill 0.6) (layers "F.Cu" "B.Cu") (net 22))
 (segment (start 40.894 -23.749001) (end 42.418 -22.225) (width 0.6) (layer "B.Cu") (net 22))
 (segment (start 42.418 -22.225) (end 42.418 -11.557) (width 0.6) (layer "B.Cu") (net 22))
 (segment (start 33.02 -9.301) (end 33.785 -8.536) (width 0.6) (layer "F.Cu") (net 18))
 (segment (start 33.02 -11.479) (end 33.02 -9.301) (width 0.6) (layer "F.Cu") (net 18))
 (segment (start 39.243 -14.478) (end 21.971 -14.478) (width 0.6) (layer "F.Cu") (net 11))
 (segment (start 40.64 -13.081) (end 39.243 -14.478) (width 0.6) (layer "F.Cu") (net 11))
 (segment (start 21.082 -15.367) (end 17.714999 -15.367) (width 0.6) (layer "F.Cu") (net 11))
 (segment (start 40.64 -11.479) (end 40.64 -13.081) (width 0.6) (layer "F.Cu") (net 11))
 (segment (start 21.971 -14.478) (end 21.082 -15.367) (width 0.6) (layer "F.Cu") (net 11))
 (segment (start 45.72 -6.731) (end 44.958 -5.969) (width 0.6) (layer "F.Cu") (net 23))
 (segment (start 42.926 -18.923) (end 45.72 -16.129) (width 0.6) (layer "F.Cu") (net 23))
 (segment (start 39.37 -19.431) (end 39.878 -18.923) (width 0.6) (layer "F.Cu") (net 23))
 (segment (start 45.72 -16.129) (end 45.72 -6.731) (width 0.6) (layer "F.Cu") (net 23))
 (segment (start 39.37 -20.779) (end 39.37 -19.431) (width 0.6) (layer "F.Cu") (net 23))
 (segment (start 39.878 -18.923) (end 42.926 -18.923) (width 0.6) (layer "F.Cu") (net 23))
 (segment (start 31.272001 -5.969) (end 28.705 -8.536001) (width 0.6) (layer "F.Cu") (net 23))
 (segment (start 44.958 -5.969) (end 31.272001 -5.969) (width 0.6) (layer "F.Cu") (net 23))
 (segment (start 38.1 -18.923) (end 39.116 -17.907) (width 0.6) (layer "F.Cu") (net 24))
 (segment (start 44.704 -7.747) (end 44.069 -7.112) (width 0.6) (layer "F.Cu") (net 24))
 (segment (start 42.418 -17.907) (end 44.704 -15.621) (width 0.6) (layer "F.Cu") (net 24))
 (segment (start 38.1 -20.779) (end 38.1 -18.923) (width 0.6) (layer "F.Cu") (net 24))
 (segment (start 44.704 -15.621) (end 44.704 -7.747) (width 0.6) (layer "F.Cu") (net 24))
 (segment (start 44.069 -7.112) (end 32.669 -7.112) (width 0.6) (layer "F.Cu") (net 24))
 (segment (start 39.116 -17.907) (end 42.418 -17.907) (width 0.6) (layer "F.Cu") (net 24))
 (segment (start 32.669 -7.112) (end 31.245001 -8.536) (width 0.6) (layer "F.Cu") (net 24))
 (segment (start 36.83 -20.778999) (end 36.83 -18.415) (width 0.6) (layer "F.Cu") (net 25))
 (segment (start 42.191 -8.536001) (end 38.865 -8.536) (width 0.6) (layer "F.Cu") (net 25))
 (segment (start 38.354 -16.891) (end 41.656 -16.891) (width 0.6) (layer "F.Cu") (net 25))
 (segment (start 43.688 -14.859) (end 43.688 -10.033) (width 0.6) (layer "F.Cu") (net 25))
 (segment (start 43.688 -10.033) (end 42.191 -8.536001) (width 0.6) (layer "F.Cu") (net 25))
 (segment (start 36.83 -18.415) (end 38.354 -16.891) (width 0.6) (layer "F.Cu") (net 25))
 (segment (start 41.656 -16.891) (end 43.688 -14.859) (width 0.6) (layer "F.Cu") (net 25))
 (segment (start 36.325001 -23.776) (end 36.325 -22.735999) (width 0.6) (layer "F.Cu") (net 26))
 (segment (start 35.56 -21.971) (end 35.56 -20.779) (width 0.6) (layer "F.Cu") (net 26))
 (segment (start 36.325 -22.735999) (end 35.56 -21.971) (width 0.6) (layer "F.Cu") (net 26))
 (segment (start 33.785 -23.776) (end 31.75 -21.741) (width 0.6) (layer "F.Cu") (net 28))
 (segment (start 31.75 -21.741) (end 31.75 -20.779) (width 0.6) (layer "F.Cu") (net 28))
 (segment (start 30.479999 -20.104761) (end 30.48 -20.778999) (width 0.6) (layer "F.Cu") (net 29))
 (segment (start 24.892 -19.431) (end 25.654 -18.669001) (width 0.6) (layer "F.Cu") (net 29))
 (segment (start 25.654 -18.669001) (end 29.044239 -18.669001) (width 0.6) (layer "F.Cu") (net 29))
 (segment (start 24.892 -22.479) (end 24.892 -19.431) (width 0.6) (layer "F.Cu") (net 29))
 (segment (start 26.165 -23.776) (end 26.165 -23.752) (width 0.6) (layer "F.Cu") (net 29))
 (segment (start 26.165 -23.752) (end 24.892 -22.479) (width 0.6) (layer "F.Cu") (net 29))
 (segment (start 29.044239 -18.669001) (end 30.479999 -20.104761) (width 0.6) (layer "F.Cu") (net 29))
 (segment (start 29.21 -21.741) (end 29.21 -20.779) (width 0.6) (layer "F.Cu") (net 30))
 (segment (start 31.245 -23.776) (end 29.21 -21.741) (width 0.6) (layer "F.Cu") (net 30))
 (segment (start 28.705 -23.776) (end 27.94 -23.011) (width 0.6) (layer "F.Cu") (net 31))
 (segment (start 27.94 -23.011) (end 27.94 -20.779) (width 0.6) (layer "F.Cu") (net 31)))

